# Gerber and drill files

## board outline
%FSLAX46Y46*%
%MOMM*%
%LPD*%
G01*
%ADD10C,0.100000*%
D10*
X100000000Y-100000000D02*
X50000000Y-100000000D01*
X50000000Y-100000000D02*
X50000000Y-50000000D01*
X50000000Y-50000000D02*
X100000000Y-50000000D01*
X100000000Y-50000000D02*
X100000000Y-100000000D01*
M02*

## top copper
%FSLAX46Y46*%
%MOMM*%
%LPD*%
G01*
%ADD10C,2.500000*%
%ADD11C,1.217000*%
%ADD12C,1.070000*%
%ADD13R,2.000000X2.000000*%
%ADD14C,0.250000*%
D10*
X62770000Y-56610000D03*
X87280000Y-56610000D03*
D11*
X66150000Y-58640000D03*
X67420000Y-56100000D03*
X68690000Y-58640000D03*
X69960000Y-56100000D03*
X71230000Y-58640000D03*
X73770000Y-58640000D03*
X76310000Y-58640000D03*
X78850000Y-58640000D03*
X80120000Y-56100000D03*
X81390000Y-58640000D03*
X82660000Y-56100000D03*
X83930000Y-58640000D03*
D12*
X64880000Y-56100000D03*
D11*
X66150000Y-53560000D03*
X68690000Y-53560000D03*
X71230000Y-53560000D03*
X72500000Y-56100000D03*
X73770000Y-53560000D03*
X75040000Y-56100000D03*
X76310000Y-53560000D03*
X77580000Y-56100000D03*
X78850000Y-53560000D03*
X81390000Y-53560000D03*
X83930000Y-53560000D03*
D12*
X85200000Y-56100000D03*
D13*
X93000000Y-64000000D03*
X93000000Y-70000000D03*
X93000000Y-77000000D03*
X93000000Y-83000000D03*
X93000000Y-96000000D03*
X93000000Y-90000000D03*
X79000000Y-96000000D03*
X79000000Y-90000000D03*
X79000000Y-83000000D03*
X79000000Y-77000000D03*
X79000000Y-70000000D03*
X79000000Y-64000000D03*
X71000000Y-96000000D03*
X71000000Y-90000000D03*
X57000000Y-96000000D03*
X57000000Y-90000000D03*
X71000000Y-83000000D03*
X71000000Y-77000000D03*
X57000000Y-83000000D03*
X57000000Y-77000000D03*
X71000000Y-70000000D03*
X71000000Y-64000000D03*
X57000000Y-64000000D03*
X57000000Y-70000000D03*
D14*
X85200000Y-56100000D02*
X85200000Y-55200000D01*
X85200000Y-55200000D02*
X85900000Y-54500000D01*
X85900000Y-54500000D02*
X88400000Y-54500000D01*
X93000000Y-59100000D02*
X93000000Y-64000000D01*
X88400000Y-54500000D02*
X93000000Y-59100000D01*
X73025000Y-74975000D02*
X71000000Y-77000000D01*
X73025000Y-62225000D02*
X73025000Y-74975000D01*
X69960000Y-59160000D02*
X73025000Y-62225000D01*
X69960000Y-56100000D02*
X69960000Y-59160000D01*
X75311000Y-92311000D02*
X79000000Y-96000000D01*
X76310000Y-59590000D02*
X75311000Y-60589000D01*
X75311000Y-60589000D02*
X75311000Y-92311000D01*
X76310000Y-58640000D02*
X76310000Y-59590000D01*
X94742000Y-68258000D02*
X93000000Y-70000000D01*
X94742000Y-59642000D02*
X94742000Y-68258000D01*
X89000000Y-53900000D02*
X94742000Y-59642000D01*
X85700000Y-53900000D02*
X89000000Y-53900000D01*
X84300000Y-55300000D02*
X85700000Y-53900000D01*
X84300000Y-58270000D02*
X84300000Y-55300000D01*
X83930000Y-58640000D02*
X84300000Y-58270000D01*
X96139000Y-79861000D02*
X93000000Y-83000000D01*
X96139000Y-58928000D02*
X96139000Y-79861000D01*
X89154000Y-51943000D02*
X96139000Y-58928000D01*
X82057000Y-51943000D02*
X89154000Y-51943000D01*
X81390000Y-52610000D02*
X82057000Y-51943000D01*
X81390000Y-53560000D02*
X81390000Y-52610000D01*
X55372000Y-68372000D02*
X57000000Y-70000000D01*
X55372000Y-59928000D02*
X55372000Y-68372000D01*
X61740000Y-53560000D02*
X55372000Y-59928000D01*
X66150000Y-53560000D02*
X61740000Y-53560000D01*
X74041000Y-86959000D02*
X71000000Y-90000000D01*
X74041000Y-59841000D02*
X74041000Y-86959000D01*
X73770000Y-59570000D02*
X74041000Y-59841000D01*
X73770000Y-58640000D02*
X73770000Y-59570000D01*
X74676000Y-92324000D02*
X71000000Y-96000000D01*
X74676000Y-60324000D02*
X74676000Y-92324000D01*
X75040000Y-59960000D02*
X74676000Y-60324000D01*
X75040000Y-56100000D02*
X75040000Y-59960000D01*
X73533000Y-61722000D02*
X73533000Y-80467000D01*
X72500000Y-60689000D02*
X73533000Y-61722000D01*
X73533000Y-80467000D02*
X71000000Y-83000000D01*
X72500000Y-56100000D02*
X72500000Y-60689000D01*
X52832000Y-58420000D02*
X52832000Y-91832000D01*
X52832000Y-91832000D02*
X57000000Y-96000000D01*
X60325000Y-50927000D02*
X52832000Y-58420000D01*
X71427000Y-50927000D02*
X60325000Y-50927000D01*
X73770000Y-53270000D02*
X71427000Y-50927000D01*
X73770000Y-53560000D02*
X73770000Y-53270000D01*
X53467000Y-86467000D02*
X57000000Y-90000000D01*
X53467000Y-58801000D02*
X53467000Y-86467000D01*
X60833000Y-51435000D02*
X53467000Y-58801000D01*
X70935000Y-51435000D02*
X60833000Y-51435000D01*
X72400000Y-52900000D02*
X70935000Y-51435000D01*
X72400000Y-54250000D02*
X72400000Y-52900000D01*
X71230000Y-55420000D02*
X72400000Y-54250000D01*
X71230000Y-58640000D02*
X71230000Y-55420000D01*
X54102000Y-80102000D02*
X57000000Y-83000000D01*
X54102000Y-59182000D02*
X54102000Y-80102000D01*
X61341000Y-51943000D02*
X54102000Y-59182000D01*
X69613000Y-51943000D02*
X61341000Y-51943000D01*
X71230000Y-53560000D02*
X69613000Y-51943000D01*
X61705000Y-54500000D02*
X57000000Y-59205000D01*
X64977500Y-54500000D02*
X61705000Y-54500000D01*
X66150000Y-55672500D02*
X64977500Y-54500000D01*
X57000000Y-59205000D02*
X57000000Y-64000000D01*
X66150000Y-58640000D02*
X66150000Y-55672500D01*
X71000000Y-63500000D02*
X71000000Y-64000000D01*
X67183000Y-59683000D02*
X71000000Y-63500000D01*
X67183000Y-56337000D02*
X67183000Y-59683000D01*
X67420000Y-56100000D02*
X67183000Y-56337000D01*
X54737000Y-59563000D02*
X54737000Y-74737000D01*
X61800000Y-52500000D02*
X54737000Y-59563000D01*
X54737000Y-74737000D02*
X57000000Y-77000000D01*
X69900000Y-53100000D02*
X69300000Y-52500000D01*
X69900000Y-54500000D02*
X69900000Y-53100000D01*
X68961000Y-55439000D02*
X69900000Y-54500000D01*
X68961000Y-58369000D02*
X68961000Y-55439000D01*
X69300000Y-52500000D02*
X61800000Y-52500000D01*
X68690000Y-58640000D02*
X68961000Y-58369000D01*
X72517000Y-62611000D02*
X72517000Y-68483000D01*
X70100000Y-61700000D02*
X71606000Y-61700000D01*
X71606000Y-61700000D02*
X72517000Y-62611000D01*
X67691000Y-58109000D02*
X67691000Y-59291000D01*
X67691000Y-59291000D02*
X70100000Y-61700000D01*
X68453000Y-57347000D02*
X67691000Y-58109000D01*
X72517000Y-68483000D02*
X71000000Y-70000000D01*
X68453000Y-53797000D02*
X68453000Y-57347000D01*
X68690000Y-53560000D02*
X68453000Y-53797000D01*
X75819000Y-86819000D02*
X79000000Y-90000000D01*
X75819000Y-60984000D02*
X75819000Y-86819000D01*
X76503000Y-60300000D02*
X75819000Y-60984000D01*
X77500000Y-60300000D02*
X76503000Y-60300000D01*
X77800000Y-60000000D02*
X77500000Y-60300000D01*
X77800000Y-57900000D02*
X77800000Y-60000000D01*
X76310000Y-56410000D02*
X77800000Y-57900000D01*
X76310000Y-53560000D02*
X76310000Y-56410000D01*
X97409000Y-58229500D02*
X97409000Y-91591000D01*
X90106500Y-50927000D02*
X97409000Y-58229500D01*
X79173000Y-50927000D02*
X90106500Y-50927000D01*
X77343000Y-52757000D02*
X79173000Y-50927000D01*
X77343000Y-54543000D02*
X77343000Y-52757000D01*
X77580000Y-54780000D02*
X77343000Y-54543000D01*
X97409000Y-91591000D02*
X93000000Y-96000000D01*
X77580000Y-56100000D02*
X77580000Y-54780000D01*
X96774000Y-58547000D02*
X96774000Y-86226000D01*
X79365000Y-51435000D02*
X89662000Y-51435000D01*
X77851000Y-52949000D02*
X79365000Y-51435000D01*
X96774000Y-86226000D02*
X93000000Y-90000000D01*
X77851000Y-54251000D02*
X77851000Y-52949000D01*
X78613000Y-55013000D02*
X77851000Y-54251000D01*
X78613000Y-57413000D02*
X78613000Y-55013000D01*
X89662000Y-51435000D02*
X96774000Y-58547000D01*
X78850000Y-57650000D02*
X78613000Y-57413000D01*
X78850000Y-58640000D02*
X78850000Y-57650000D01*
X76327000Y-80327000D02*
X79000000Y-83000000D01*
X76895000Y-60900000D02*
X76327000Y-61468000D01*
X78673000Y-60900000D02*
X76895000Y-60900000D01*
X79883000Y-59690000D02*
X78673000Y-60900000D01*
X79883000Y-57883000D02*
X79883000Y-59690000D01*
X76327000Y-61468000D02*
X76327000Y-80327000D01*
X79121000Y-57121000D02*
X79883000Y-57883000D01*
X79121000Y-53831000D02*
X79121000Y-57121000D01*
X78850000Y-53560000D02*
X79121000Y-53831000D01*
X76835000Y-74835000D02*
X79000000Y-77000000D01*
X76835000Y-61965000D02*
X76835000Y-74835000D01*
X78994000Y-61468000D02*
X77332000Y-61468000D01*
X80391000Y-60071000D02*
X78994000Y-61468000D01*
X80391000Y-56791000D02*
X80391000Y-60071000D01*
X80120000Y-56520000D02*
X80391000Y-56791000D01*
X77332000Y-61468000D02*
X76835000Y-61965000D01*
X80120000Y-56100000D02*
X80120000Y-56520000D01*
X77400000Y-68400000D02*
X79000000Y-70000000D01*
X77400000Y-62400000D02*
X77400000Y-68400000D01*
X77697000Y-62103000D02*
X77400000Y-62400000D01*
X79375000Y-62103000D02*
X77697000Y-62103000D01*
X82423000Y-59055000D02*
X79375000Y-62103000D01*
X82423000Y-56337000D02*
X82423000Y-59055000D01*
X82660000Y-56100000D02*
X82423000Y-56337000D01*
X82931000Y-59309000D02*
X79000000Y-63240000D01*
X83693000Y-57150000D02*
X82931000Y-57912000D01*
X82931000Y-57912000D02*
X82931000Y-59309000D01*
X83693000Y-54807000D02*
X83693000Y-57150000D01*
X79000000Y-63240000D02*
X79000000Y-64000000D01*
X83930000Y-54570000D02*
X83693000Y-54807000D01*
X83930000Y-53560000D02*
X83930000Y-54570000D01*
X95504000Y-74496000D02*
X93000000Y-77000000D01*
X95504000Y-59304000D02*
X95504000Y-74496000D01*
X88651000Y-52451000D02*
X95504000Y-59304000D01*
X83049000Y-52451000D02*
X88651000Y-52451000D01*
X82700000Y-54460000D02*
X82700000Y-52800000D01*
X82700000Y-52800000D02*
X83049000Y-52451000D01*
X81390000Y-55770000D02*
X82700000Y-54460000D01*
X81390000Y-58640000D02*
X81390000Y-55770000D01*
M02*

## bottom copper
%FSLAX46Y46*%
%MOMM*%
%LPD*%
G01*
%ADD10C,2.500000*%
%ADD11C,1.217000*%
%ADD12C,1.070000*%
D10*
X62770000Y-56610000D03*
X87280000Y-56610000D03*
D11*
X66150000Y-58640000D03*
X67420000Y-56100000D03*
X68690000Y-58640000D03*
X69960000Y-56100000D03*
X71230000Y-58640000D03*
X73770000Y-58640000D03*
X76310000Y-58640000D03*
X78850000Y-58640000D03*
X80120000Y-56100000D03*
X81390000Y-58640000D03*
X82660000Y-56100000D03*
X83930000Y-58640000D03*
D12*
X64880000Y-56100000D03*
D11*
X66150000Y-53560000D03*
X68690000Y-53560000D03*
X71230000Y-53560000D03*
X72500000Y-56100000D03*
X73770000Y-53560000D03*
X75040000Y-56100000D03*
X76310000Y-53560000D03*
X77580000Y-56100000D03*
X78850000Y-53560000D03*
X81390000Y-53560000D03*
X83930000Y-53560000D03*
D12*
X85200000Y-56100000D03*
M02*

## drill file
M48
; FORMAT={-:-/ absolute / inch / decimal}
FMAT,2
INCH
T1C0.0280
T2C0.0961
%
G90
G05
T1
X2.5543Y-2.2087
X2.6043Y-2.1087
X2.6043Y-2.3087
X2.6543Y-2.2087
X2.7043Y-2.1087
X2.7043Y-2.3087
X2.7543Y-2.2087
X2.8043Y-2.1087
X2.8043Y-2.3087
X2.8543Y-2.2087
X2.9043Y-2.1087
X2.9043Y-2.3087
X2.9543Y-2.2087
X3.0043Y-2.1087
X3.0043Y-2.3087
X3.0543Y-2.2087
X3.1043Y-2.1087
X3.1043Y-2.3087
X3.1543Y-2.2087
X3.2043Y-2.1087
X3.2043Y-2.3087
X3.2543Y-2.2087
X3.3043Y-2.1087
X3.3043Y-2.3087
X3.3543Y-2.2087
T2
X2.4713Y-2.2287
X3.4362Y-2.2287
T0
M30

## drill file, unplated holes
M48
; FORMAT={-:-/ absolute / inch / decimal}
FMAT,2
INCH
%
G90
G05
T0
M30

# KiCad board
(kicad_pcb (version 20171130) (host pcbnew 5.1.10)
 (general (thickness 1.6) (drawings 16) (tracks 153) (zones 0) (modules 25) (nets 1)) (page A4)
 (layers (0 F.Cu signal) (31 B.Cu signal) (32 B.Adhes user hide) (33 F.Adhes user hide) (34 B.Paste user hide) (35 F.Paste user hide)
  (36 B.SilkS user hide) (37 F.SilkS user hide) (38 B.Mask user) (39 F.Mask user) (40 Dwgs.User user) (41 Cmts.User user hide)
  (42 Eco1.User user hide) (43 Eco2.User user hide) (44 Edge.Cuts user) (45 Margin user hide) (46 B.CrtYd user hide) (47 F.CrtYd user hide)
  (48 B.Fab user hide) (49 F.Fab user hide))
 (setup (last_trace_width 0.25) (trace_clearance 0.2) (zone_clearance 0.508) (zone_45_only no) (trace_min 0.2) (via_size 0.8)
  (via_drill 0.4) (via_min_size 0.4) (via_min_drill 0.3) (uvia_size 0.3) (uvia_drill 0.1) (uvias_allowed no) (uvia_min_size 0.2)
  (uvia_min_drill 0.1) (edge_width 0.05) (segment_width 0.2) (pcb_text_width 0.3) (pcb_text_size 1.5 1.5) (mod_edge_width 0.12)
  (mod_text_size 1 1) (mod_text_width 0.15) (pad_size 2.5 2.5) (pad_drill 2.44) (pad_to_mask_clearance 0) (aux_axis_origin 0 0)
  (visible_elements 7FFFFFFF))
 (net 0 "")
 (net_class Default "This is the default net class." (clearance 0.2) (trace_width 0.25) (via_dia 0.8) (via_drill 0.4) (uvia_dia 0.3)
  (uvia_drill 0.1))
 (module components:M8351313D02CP (layer F.Cu) (at 85.2 56.1)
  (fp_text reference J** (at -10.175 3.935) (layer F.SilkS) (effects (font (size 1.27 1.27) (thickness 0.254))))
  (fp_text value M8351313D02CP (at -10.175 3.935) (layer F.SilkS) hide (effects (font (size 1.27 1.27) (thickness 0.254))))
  (pad MH2 thru_hole circle (at -22.43 0.51) (size 2.5 2.5) (drill 2.44) (layers *.Cu *.Mask))
  (pad MH1 thru_hole circle (at 2.08 0.51) (size 2.5 2.5) (drill 2.44) (layers *.Cu *.Mask))
  (pad 25 thru_hole circle (at -19.05 2.54) (size 1.217 1.217) (drill 0.71) (layers *.Cu *.Mask))
  (pad 24 thru_hole circle (at -17.78 0) (size 1.217 1.217) (drill 0.71) (layers *.Cu *.Mask))
  (pad 23 thru_hole circle (at -16.51 2.54) (size 1.217 1.217) (drill 0.71) (layers *.Cu *.Mask))
  (pad 22 thru_hole circle (at -15.24 0) (size 1.217 1.217) (drill 0.71) (layers *.Cu *.Mask))
  (pad 21 thru_hole circle (at -13.97 2.54) (size 1.217 1.217) (drill 0.71) (layers *.Cu *.Mask))
  (pad 20 thru_hole circle (at -11.43 2.54) (size 1.217 1.217) (drill 0.71) (layers *.Cu *.Mask))
  (pad 19 thru_hole circle (at -8.89 2.54) (size 1.217 1.217) (drill 0.71) (layers *.Cu *.Mask))
  (pad 18 thru_hole circle (at -6.35 2.54) (size 1.217 1.217) (drill 0.71) (layers *.Cu *.Mask))
  (pad 17 thru_hole circle (at -5.08 0) (size 1.217 1.217) (drill 0.71) (layers *.Cu *.Mask))
  (pad 16 thru_hole circle (at -3.81 2.54) (size 1.217 1.217) (drill 0.71) (layers *.Cu *.Mask))
  (pad 15 thru_hole circle (at -2.54 0) (size 1.217 1.217) (drill 0.71) (layers *.Cu *.Mask))
  (pad 14 thru_hole circle (at -1.27 2.54) (size 1.217 1.217) (drill 0.71) (layers *.Cu *.Mask))
  (pad 13 thru_hole circle (at -20.32 0) (size 1.07 1.07) (drill 0.71) (layers *.Cu *.Mask))
  (pad 12 thru_hole circle (at -19.05 -2.54) (size 1.217 1.217) (drill 0.71) (layers *.Cu *.Mask))
  (pad 11 thru_hole circle (at -16.51 -2.54) (size 1.217 1.217) (drill 0.71) (layers *.Cu *.Mask))
  (pad 10 thru_hole circle (at -13.97 -2.54) (size 1.217 1.217) (drill 0.71) (layers *.Cu *.Mask))
  (pad 9 thru_hole circle (at -12.7 0) (size 1.217 1.217) (drill 0.71) (layers *.Cu *.Mask))
  (pad 8 thru_hole circle (at -11.43 -2.54) (size 1.217 1.217) (drill 0.71) (layers *.Cu *.Mask))
  (pad 7 thru_hole circle (at -10.16 0) (size 1.217 1.217) (drill 0.71) (layers *.Cu *.Mask))
  (pad 6 thru_hole circle (at -8.89 -2.54) (size 1.217 1.217) (drill 0.71) (layers *.Cu *.Mask))
  (pad 5 thru_hole circle (at -7.62 0) (size 1.217 1.217) (drill 0.71) (layers *.Cu *.Mask))
  (pad 4 thru_hole circle (at -6.35 -2.54) (size 1.217 1.217) (drill 0.71) (layers *.Cu *.Mask))
  (pad 3 thru_hole circle (at -3.81 -2.54) (size 1.217 1.217) (drill 0.71) (layers *.Cu *.Mask))
  (pad 2 thru_hole circle (at -1.27 -2.54) (size 1.217 1.217) (drill 0.71) (layers *.Cu *.Mask))
  (pad 1 thru_hole circle (at 0 0) (size 1.07 1.07) (drill 0.71) (layers *.Cu *.Mask)))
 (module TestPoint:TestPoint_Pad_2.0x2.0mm (layer F.Cu) (at 93 64)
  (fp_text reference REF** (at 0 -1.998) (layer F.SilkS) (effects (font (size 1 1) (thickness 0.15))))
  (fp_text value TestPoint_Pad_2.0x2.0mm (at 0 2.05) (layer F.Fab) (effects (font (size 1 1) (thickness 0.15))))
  (pad 1 smd rect (at 0 0) (size 2 2) (layers F.Cu F.Mask)))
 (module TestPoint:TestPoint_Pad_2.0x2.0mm (layer F.Cu) (at 93 70)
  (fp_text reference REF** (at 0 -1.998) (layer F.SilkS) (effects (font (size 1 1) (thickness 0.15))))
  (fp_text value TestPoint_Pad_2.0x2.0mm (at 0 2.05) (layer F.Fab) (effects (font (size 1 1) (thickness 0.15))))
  (pad 2 smd rect (at 0 0) (size 2 2) (layers F.Cu F.Mask)))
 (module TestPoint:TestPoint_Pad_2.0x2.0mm (layer F.Cu) (at 93 77)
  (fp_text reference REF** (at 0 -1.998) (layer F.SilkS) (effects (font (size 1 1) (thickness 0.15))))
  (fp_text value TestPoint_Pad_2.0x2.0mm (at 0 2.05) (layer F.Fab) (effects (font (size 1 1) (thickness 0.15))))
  (pad 6 smd rect (at 0 0) (size 2 2) (layers F.Cu F.Mask)))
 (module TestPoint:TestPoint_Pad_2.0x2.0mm (layer F.Cu) (at 93 83)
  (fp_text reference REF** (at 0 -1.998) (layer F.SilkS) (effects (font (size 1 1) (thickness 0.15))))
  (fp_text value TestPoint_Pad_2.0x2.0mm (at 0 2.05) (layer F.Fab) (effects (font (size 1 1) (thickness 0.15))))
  (pad 5 smd rect (at 0 0) (size 2 2) (layers F.Cu F.Mask)))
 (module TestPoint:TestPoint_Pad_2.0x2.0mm (layer F.Cu) (at 93 96)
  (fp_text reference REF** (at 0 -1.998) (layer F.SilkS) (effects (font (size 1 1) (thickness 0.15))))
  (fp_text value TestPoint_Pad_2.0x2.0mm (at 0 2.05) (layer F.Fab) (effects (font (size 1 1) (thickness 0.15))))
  (pad 9 smd rect (at 0 0) (size 2 2) (layers F.Cu F.Mask)))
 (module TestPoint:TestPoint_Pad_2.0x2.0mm (layer F.Cu) (at 93 90)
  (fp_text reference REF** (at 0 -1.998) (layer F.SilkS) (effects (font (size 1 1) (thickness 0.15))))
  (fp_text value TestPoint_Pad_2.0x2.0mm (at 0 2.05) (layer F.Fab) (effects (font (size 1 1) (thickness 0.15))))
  (pad 10 smd rect (at 0 0) (size 2 2) (layers F.Cu F.Mask)))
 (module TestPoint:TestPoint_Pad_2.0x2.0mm (layer F.Cu) (at 79 96)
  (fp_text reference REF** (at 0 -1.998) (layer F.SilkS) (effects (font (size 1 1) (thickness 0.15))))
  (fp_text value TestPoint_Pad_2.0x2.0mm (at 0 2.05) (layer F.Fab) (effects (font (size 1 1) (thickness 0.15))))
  (pad 12 smd rect (at 0 0) (size 2 2) (layers F.Cu F.Mask)))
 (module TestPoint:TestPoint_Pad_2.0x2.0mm (layer F.Cu) (at 79 90)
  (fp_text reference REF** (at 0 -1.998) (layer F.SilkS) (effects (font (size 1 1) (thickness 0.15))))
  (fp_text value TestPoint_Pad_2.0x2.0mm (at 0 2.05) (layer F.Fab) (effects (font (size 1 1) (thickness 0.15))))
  (pad 11 smd rect (at 0 0) (size 2 2) (layers F.Cu F.Mask)))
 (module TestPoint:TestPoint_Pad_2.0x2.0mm (layer F.Cu) (at 79 83)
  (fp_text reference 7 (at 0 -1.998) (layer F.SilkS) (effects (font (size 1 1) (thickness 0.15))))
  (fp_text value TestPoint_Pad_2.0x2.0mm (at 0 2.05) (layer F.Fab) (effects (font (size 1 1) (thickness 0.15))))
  (pad 7 smd rect (at 0 0) (size 2 2) (layers F.Cu F.Mask)))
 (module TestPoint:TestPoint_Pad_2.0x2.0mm (layer F.Cu) (at 79 77)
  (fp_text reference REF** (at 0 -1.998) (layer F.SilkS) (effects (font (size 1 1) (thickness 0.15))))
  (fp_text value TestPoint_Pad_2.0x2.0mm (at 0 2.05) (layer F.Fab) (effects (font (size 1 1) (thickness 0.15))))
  (pad 8 smd rect (at 0 0) (size 2 2) (layers F.Cu F.Mask)))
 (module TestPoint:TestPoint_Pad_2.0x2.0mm (layer F.Cu) (at 79 70)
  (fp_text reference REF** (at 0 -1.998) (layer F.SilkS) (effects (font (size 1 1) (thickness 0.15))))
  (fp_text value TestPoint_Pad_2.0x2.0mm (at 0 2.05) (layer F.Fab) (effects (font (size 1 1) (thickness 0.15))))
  (pad 4 smd rect (at 0 0) (size 2 2) (layers F.Cu F.Mask)))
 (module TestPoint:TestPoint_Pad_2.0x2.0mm (layer F.Cu) (at 79 64)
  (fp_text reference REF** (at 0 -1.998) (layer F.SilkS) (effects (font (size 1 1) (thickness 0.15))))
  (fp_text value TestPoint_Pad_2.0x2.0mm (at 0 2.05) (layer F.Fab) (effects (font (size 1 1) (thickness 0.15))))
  (pad 3 smd rect (at 0 0) (size 2 2) (layers F.Cu F.Mask)))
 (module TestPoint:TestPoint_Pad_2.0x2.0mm (layer F.Cu) (at 71 96)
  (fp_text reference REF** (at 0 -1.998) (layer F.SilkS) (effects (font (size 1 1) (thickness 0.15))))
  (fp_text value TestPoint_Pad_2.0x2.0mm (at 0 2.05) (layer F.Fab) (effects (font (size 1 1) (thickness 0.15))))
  (pad 13 smd rect (at 0 0) (size 2 2) (layers F.Cu F.Mask)))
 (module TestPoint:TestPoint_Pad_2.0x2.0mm (layer F.Cu) (at 71 90)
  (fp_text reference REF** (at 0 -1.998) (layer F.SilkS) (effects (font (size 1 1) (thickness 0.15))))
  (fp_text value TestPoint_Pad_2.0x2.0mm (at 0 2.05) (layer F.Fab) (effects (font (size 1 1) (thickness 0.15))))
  (pad 14 smd rect (at 0 0) (size 2 2) (layers F.Cu F.Mask)))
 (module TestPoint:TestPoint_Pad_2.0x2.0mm (layer F.Cu) (at 57 96)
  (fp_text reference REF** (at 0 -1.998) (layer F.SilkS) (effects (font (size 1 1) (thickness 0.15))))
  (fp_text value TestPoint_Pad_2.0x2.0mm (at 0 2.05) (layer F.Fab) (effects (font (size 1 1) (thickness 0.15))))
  (pad 15 smd rect (at 0 0) (size 2 2) (layers F.Cu F.Mask)))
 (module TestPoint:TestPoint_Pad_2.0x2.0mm (layer F.Cu) (at 57 90)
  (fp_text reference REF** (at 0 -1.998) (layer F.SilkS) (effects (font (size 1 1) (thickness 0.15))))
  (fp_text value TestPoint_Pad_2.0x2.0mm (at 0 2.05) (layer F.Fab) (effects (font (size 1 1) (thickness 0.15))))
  (pad 16 smd rect (at 0 0) (size 2 2) (layers F.Cu F.Mask)))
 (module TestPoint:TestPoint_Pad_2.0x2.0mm (layer F.Cu) (at 71 83)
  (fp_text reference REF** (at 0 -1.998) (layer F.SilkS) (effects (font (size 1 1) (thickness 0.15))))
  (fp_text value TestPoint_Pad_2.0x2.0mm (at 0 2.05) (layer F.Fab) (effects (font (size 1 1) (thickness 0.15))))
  (pad 17 smd rect (at 0 0) (size 2 2) (layers F.Cu F.Mask)))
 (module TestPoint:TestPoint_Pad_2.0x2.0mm (layer F.Cu) (at 71 77)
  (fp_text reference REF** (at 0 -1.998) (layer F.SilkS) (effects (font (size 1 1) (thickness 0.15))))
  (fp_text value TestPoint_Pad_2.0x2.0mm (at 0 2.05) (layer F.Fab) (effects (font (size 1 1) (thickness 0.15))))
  (pad 18 smd rect (at 0 0) (size 2 2) (layers F.Cu F.Mask)))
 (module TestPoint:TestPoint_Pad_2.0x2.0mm (layer F.Cu) (at 57 83)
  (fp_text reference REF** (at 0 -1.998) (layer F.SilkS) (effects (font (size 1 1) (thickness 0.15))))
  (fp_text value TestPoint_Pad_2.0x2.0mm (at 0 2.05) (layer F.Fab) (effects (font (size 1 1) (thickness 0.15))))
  (pad 19 smd rect (at 0 0) (size 2 2) (layers F.Cu F.Mask)))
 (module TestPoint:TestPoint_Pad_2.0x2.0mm (layer F.Cu) (at 57 77)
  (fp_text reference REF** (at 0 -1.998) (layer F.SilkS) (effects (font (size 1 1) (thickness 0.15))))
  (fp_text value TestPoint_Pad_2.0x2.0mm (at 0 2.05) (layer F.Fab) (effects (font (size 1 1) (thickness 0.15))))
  (pad 20 smd rect (at 0 0) (size 2 2) (layers F.Cu F.Mask)))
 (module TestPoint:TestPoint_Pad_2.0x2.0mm (layer F.Cu) (at 71 70)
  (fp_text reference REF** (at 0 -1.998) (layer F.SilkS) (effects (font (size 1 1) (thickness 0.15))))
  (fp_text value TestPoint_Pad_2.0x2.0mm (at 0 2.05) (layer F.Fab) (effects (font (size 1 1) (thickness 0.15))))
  (pad 21 smd rect (at 0 0) (size 2 2) (layers F.Cu F.Mask)))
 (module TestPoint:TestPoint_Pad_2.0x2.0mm (layer F.Cu) (at 71 64)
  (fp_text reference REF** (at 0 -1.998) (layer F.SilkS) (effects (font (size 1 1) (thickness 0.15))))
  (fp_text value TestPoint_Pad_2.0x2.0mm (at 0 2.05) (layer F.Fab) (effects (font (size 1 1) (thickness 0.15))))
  (pad 22 smd rect (at 0 0) (size 2 2) (layers F.Cu F.Mask)))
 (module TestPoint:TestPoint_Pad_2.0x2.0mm (layer F.Cu) (at 57 64)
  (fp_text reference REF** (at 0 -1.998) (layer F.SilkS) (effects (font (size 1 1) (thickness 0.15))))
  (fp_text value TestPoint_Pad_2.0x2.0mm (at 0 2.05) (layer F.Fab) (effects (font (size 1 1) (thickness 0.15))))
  (pad 24 smd rect (at 0 0) (size 2 2) (layers F.Cu F.Mask)))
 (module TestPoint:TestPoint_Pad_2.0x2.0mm (layer F.Cu) (at 57 70)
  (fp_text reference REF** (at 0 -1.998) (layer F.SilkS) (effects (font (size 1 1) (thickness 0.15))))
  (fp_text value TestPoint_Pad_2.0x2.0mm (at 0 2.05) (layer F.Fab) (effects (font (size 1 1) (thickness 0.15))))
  (pad 23 smd rect (at 0 0) (size 2 2) (layers F.Cu F.Mask)))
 (gr_poly (pts (xy 100 100) (xy 50 100) (xy 50 50) (xy 100 50)) (layer Edge.Cuts) (width 0.1))
 (segment (start 85.2 56.1) (end 85.2 55.2) (width 0.25) (layer F.Cu) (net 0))
 (segment (start 85.2 55.2) (end 85.9 54.5) (width 0.25) (layer F.Cu) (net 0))
 (segment (start 85.9 54.5) (end 88.4 54.5) (width 0.25) (layer F.Cu) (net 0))
 (segment (start 93 59.1) (end 93 64) (width 0.25) (layer F.Cu) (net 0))
 (segment (start 88.4 54.5) (end 93 59.1) (width 0.25) (layer F.Cu) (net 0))
 (segment (start 73.025 74.975) (end 71 77) (width 0.25) (layer F.Cu) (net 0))
 (segment (start 73.025 62.225) (end 73.025 74.975) (width 0.25) (layer F.Cu) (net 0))
 (segment (start 69.96 59.16) (end 73.025 62.225) (width 0.25) (layer F.Cu) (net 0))
 (segment (start 69.96 56.1) (end 69.96 59.16) (width 0.25) (layer F.Cu) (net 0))
 (segment (start 75.311 92.311) (end 79 96) (width 0.25) (layer F.Cu) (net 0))
 (segment (start 76.31 59.59) (end 75.311 60.589) (width 0.25) (layer F.Cu) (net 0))
 (segment (start 75.311 60.589) (end 75.311 92.311) (width 0.25) (layer F.Cu) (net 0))
 (segment (start 76.31 58.64) (end 76.31 59.59) (width 0.25) (layer F.Cu) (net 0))
 (segment (start 94.742 68.258) (end 93 70) (width 0.25) (layer F.Cu) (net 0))
 (segment (start 94.742 59.642) (end 94.742 68.258) (width 0.25) (layer F.Cu) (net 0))
 (segment (start 89 53.9) (end 94.742 59.642) (width 0.25) (layer F.Cu) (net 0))
 (segment (start 85.7 53.9) (end 89 53.9) (width 0.25) (layer F.Cu) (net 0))
 (segment (start 84.3 55.3) (end 85.7 53.9) (width 0.25) (layer F.Cu) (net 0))
 (segment (start 84.3 58.27) (end 84.3 55.3) (width 0.25) (layer F.Cu) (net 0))
 (segment (start 83.93 58.64) (end 84.3 58.27) (width 0.25) (layer F.Cu) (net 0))
 (segment (start 96.139 79.861) (end 93 83) (width 0.25) (layer F.Cu) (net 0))
 (segment (start 96.139 58.928) (end 96.139 79.861) (width 0.25) (layer F.Cu) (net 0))
 (segment (start 89.154 51.943) (end 96.139 58.928) (width 0.25) (layer F.Cu) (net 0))
 (segment (start 82.057 51.943) (end 89.154 51.943) (width 0.25) (layer F.Cu) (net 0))
 (segment (start 81.39 52.61) (end 82.057 51.943) (width 0.25) (layer F.Cu) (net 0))
 (segment (start 81.39 53.56) (end 81.39 52.61) (width 0.25) (layer F.Cu) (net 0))
 (segment (start 55.372 68.372) (end 57 70) (width 0.25) (layer F.Cu) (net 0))
 (segment (start 55.372 59.928) (end 55.372 68.372) (width 0.25) (layer F.Cu) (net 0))
 (segment (start 61.74 53.56) (end 55.372 59.928) (width 0.25) (layer F.Cu) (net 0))
 (segment (start 66.15 53.56) (end 61.74 53.56) (width 0.25) (layer F.Cu) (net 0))
 (segment (start 74.041 86.959) (end 71 90) (width 0.25) (layer F.Cu) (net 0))
 (segment (start 74.041 59.841) (end 74.041 86.959) (width 0.25) (layer F.Cu) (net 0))
 (segment (start 73.77 59.57) (end 74.041 59.841) (width 0.25) (layer F.Cu) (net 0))
 (segment (start 73.77 58.64) (end 73.77 59.57) (width 0.25) (layer F.Cu) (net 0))
 (segment (start 74.676 92.324) (end 71 96) (width 0.25) (layer F.Cu) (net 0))
 (segment (start 74.676 60.324) (end 74.676 92.324) (width 0.25) (layer F.Cu) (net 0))
 (segment (start 75.04 59.96) (end 74.676 60.324) (width 0.25) (layer F.Cu) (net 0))
 (segment (start 75.04 56.1) (end 75.04 59.96) (width 0.25) (layer F.Cu) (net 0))
 (segment (start 73.533 61.722) (end 73.533 80.467) (width 0.25) (layer F.Cu) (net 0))
 (segment (start 72.5 60.689) (end 73.533 61.722) (width 0.25) (layer F.Cu) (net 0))
 (segment (start 73.533 80.467) (end 71 83) (width 0.25) (layer F.Cu) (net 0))
 (segment (start 72.5 56.1) (end 72.5 60.689) (width 0.25) (layer F.Cu) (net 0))
 (segment (start 52.832 58.42) (end 52.832 91.832) (width 0.25) (layer F.Cu) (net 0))
 (segment (start 52.832 91.832) (end 57 96) (width 0.25) (layer F.Cu) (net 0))
 (segment (start 60.325 50.927) (end 52.832 58.42) (width 0.25) (layer F.Cu) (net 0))
 (segment (start 71.427 50.927) (end 60.325 50.927) (width 0.25) (layer F.Cu) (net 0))
 (segment (start 73.77 53.27) (end 71.427 50.927) (width 0.25) (layer F.Cu) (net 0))
 (segment (start 73.77 53.56) (end 73.77 53.27) (width 0.25) (layer F.Cu) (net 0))
 (segment (start 53.467 86.467) (end 57 90) (width 0.25) (layer F.Cu) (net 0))
 (segment (start 53.467 58.801) (end 53.467 86.467) (width 0.25) (layer F.Cu) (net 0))
 (segment (start 60.833 51.435) (end 53.467 58.801) (width 0.25) (layer F.Cu) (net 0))
 (segment (start 70.935 51.435) (end 60.833 51.435) (width 0.25) (layer F.Cu) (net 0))
 (segment (start 72.4 52.9) (end 70.935 51.435) (width 0.25) (layer F.Cu) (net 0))
 (segment (start 72.4 54.25) (end 72.4 52.9) (width 0.25) (layer F.Cu) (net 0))
 (segment (start 71.23 55.42) (end 72.4 54.25) (width 0.25) (layer F.Cu) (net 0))
 (segment (start 71.23 58.64) (end 71.23 55.42) (width 0.25) (layer F.Cu) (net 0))
 (segment (start 54.102 80.102) (end 57 83) (width 0.25) (layer F.Cu) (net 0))
 (segment (start 54.102 59.182) (end 54.102 80.102) (width 0.25) (layer F.Cu) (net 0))
 (segment (start 61.341 51.943) (end 54.102 59.182) (width 0.25) (layer F.Cu) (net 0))
 (segment (start 69.613 51.943) (end 61.341 51.943) (width 0.25) (layer F.Cu) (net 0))
 (segment (start 71.23 53.56) (end 69.613 51.943) (width 0.25) (layer F.Cu) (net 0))
 (segment (start 61.705 54.5) (end 57 59.205) (width 0.25) (layer F.Cu) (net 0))
 (segment (start 64.9775 54.5) (end 61.705 54.5) (width 0.25) (layer F.Cu) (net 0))
 (segment (start 66.15 55.6725) (end 64.9775 54.5) (width 0.25) (layer F.Cu) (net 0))
 (segment (start 57 59.205) (end 57 64) (width 0.25) (layer F.Cu) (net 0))
 (segment (start 66.15 58.64) (end 66.15 55.6725) (width 0.25) (layer F.Cu) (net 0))
 (segment (start 71 63.5) (end 71 64) (width 0.25) (layer F.Cu) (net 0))
 (segment (start 67.183 59.683) (end 71 63.5) (width 0.25) (layer F.Cu) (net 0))
 (segment (start 67.183 56.337) (end 67.183 59.683) (width 0.25) (layer F.Cu) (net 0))
 (segment (start 67.42 56.1) (end 67.183 56.337) (width 0.25) (layer F.Cu) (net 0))
 (segment (start 54.737 59.563) (end 54.737 74.737) (width 0.25) (layer F.Cu) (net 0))
 (segment (start 61.8 52.5) (end 54.737 59.563) (width 0.25) (layer F.Cu) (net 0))
 (segment (start 54.737 74.737) (end 57 77) (width 0.25) (layer F.Cu) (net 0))
 (segment (start 69.9 53.1) (end 69.3 52.5) (width 0.25) (layer F.Cu) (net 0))
 (segment (start 69.9 54.5) (end 69.9 53.1) (width 0.25) (layer F.Cu) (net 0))
 (segment (start 68.961 55.439) (end 69.9 54.5) (width 0.25) (layer F.Cu) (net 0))
 (segment (start 68.961 58.369) (end 68.961 55.439) (width 0.25) (layer F.Cu) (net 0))
 (segment (start 69.3 52.5) (end 61.8 52.5) (width 0.25) (layer F.Cu) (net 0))
 (segment (start 68.69 58.64) (end 68.961 58.369) (width 0.25) (layer F.Cu) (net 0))
 (segment (start 72.517 62.611) (end 72.517 68.483) (width 0.25) (layer F.Cu) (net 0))
 (segment (start 70.1 61.7) (end 71.606 61.7) (width 0.25) (layer F.Cu) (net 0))
 (segment (start 71.606 61.7) (end 72.517 62.611) (width 0.25) (layer F.Cu) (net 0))
 (segment (start 67.691 58.109) (end 67.691 59.291) (width 0.25) (layer F.Cu) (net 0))
 (segment (start 67.691 59.291) (end 70.1 61.7) (width 0.25) (layer F.Cu) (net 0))
 (segment (start 68.453 57.347) (end 67.691 58.109) (width 0.25) (layer F.Cu) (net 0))
 (segment (start 72.517 68.483) (end 71 70) (width 0.25) (layer F.Cu) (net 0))
 (segment (start 68.453 53.797) (end 68.453 57.347) (width 0.25) (layer F.Cu) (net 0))
 (segment (start 68.69 53.56) (end 68.453 53.797) (width 0.25) (layer F.Cu) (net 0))
 (segment (start 75.819 86.819) (end 79 90) (width 0.25) (layer F.Cu) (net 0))
 (segment (start 75.819 60.984) (end 75.819 86.819) (width 0.25) (layer F.Cu) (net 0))
 (segment (start 76.503 60.3) (end 75.819 60.984) (width 0.25) (layer F.Cu) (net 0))
 (segment (start 77.5 60.3) (end 76.503 60.3) (width 0.25) (layer F.Cu) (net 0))
 (segment (start 77.8 60) (end 77.5 60.3) (width 0.25) (layer F.Cu) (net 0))
 (segment (start 77.8 57.9) (end 77.8 60) (width 0.25) (layer F.Cu) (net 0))
 (segment (start 76.31 56.41) (end 77.8 57.9) (width 0.25) (layer F.Cu) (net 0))
 (segment (start 76.31 53.56) (end 76.31 56.41) (width 0.25) (layer F.Cu) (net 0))
 (segment (start 97.409 58.2295) (end 97.409 91.591) (width 0.25) (layer F.Cu) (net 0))
 (segment (start 90.1065 50.927) (end 97.409 58.2295) (width 0.25) (layer F.Cu) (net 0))
 (segment (start 79.173 50.927) (end 90.1065 50.927) (width 0.25) (layer F.Cu) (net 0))
 (segment (start 77.343 52.757) (end 79.173 50.927) (width 0.25) (layer F.Cu) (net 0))
 (segment (start 77.343 54.543) (end 77.343 52.757) (width 0.25) (layer F.Cu) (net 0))
 (segment (start 77.58 54.78) (end 77.343 54.543) (width 0.25) (layer F.Cu) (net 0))
 (segment (start 97.409 91.591) (end 93 96) (width 0.25) (layer F.Cu) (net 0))
 (segment (start 77.58 56.1) (end 77.58 54.78) (width 0.25) (layer F.Cu) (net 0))
 (segment (start 96.774 58.547) (end 96.774 86.226) (width 0.25) (layer F.Cu) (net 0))
 (segment (start 79.365 51.435) (end 89.662 51.435) (width 0.25) (layer F.Cu) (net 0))
 (segment (start 77.851 52.949) (end 79.365 51.435) (width 0.25) (layer F.Cu) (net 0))
 (segment (start 96.774 86.226) (end 93 90) (width 0.25) (layer F.Cu) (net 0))
 (segment (start 77.851 54.251) (end 77.851 52.949) (width 0.25) (layer F.Cu) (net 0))
 (segment (start 78.613 55.013) (end 77.851 54.251) (width 0.25) (layer F.Cu) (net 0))
 (segment (start 78.613 57.413) (end 78.613 55.013) (width 0.25) (layer F.Cu) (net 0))
 (segment (start 89.662 51.435) (end 96.774 58.547) (width 0.25) (layer F.Cu) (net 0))
 (segment (start 78.85 57.65) (end 78.613 57.413) (width 0.25) (layer F.Cu) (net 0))
 (segment (start 78.85 58.64) (end 78.85 57.65) (width 0.25) (layer F.Cu) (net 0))
 (segment (start 76.327 80.327) (end 79 83) (width 0.25) (layer F.Cu) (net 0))
 (segment (start 76.895 60.9) (end 76.327 61.468) (width 0.25) (layer F.Cu) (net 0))
 (segment (start 78.673 60.9) (end 76.895 60.9) (width 0.25) (layer F.Cu) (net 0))
 (segment (start 79.883 59.69) (end 78.673 60.9) (width 0.25) (layer F.Cu) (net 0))
 (segment (start 79.883 57.883) (end 79.883 59.69) (width 0.25) (layer F.Cu) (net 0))
 (segment (start 76.327 61.468) (end 76.327 80.327) (width 0.25) (layer F.Cu) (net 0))
 (segment (start 79.121 57.121) (end 79.883 57.883) (width 0.25) (layer F.Cu) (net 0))
 (segment (start 79.121 53.831) (end 79.121 57.121) (width 0.25) (layer F.Cu) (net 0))
 (segment (start 78.85 53.56) (end 79.121 53.831) (width 0.25) (layer F.Cu) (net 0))
 (segment (start 76.835 74.835) (end 79 77) (width 0.25) (layer F.Cu) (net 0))
 (segment (start 76.835 61.965) (end 76.835 74.835) (width 0.25) (layer F.Cu) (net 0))
 (segment (start 78.994 61.468) (end 77.332 61.468) (width 0.25) (layer F.Cu) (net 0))
 (segment (start 80.391 60.071) (end 78.994 61.468) (width 0.25) (layer F.Cu) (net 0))
 (segment (start 80.391 56.791) (end 80.391 60.071) (width 0.25) (layer F.Cu) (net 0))
 (segment (start 80.12 56.52) (end 80.391 56.791) (width 0.25) (layer F.Cu) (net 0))
 (segment (start 77.332 61.468) (end 76.835 61.965) (width 0.25) (layer F.Cu) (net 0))
 (segment (start 80.12 56.1) (end 80.12 56.52) (width 0.25) (layer F.Cu) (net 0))
 (segment (start 77.4 68.4) (end 79 70) (width 0.25) (layer F.Cu) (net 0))
 (segment (start 77.4 62.4) (end 77.4 68.4) (width 0.25) (layer F.Cu) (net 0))
 (segment (start 77.697 62.103) (end 77.4 62.4) (width 0.25) (layer F.Cu) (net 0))
 (segment (start 79.375 62.103) (end 77.697 62.103) (width 0.25) (layer F.Cu) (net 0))
 (segment (start 82.423 59.055) (end 79.375 62.103) (width 0.25) (layer F.Cu) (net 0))
 (segment (start 82.423 56.337) (end 82.423 59.055) (width 0.25) (layer F.Cu) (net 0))
 (segment (start 82.66 56.1) (end 82.423 56.337) (width 0.25) (layer F.Cu) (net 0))
 (segment (start 82.931 59.309) (end 79 63.24) (width 0.25) (layer F.Cu) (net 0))
 (segment (start 83.693 57.15) (end 82.931 57.912) (width 0.25) (layer F.Cu) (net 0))
 (segment (start 82.931 57.912) (end 82.931 59.309) (width 0.25) (layer F.Cu) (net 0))
 (segment (start 83.693 54.807) (end 83.693 57.15) (width 0.25) (layer F.Cu) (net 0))
 (segment (start 79 63.24) (end 79 64) (width 0.25) (layer F.Cu) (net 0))
 (segment (start 83.93 54.57) (end 83.693 54.807) (width 0.25) (layer F.Cu) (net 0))
 (segment (start 83.93 53.56) (end 83.93 54.57) (width 0.25) (layer F.Cu) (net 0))
 (segment (start 95.504 74.496) (end 93 77) (width 0.25) (layer F.Cu) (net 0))
 (segment (start 95.504 59.304) (end 95.504 74.496) (width 0.25) (layer F.Cu) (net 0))
 (segment (start 88.651 52.451) (end 95.504 59.304) (width 0.25) (layer F.Cu) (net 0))
 (segment (start 83.049 52.451) (end 88.651 52.451) (width 0.25) (layer F.Cu) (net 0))
 (segment (start 82.7 54.46) (end 82.7 52.8) (width 0.25) (layer F.Cu) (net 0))
 (segment (start 82.7 52.8) (end 83.049 52.451) (width 0.25) (layer F.Cu) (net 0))
 (segment (start 81.39 55.77) (end 82.7 54.46) (width 0.25) (layer F.Cu) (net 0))
 (segment (start 81.39 58.64) (end 81.39 55.77) (width 0.25) (layer F.Cu) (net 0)))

